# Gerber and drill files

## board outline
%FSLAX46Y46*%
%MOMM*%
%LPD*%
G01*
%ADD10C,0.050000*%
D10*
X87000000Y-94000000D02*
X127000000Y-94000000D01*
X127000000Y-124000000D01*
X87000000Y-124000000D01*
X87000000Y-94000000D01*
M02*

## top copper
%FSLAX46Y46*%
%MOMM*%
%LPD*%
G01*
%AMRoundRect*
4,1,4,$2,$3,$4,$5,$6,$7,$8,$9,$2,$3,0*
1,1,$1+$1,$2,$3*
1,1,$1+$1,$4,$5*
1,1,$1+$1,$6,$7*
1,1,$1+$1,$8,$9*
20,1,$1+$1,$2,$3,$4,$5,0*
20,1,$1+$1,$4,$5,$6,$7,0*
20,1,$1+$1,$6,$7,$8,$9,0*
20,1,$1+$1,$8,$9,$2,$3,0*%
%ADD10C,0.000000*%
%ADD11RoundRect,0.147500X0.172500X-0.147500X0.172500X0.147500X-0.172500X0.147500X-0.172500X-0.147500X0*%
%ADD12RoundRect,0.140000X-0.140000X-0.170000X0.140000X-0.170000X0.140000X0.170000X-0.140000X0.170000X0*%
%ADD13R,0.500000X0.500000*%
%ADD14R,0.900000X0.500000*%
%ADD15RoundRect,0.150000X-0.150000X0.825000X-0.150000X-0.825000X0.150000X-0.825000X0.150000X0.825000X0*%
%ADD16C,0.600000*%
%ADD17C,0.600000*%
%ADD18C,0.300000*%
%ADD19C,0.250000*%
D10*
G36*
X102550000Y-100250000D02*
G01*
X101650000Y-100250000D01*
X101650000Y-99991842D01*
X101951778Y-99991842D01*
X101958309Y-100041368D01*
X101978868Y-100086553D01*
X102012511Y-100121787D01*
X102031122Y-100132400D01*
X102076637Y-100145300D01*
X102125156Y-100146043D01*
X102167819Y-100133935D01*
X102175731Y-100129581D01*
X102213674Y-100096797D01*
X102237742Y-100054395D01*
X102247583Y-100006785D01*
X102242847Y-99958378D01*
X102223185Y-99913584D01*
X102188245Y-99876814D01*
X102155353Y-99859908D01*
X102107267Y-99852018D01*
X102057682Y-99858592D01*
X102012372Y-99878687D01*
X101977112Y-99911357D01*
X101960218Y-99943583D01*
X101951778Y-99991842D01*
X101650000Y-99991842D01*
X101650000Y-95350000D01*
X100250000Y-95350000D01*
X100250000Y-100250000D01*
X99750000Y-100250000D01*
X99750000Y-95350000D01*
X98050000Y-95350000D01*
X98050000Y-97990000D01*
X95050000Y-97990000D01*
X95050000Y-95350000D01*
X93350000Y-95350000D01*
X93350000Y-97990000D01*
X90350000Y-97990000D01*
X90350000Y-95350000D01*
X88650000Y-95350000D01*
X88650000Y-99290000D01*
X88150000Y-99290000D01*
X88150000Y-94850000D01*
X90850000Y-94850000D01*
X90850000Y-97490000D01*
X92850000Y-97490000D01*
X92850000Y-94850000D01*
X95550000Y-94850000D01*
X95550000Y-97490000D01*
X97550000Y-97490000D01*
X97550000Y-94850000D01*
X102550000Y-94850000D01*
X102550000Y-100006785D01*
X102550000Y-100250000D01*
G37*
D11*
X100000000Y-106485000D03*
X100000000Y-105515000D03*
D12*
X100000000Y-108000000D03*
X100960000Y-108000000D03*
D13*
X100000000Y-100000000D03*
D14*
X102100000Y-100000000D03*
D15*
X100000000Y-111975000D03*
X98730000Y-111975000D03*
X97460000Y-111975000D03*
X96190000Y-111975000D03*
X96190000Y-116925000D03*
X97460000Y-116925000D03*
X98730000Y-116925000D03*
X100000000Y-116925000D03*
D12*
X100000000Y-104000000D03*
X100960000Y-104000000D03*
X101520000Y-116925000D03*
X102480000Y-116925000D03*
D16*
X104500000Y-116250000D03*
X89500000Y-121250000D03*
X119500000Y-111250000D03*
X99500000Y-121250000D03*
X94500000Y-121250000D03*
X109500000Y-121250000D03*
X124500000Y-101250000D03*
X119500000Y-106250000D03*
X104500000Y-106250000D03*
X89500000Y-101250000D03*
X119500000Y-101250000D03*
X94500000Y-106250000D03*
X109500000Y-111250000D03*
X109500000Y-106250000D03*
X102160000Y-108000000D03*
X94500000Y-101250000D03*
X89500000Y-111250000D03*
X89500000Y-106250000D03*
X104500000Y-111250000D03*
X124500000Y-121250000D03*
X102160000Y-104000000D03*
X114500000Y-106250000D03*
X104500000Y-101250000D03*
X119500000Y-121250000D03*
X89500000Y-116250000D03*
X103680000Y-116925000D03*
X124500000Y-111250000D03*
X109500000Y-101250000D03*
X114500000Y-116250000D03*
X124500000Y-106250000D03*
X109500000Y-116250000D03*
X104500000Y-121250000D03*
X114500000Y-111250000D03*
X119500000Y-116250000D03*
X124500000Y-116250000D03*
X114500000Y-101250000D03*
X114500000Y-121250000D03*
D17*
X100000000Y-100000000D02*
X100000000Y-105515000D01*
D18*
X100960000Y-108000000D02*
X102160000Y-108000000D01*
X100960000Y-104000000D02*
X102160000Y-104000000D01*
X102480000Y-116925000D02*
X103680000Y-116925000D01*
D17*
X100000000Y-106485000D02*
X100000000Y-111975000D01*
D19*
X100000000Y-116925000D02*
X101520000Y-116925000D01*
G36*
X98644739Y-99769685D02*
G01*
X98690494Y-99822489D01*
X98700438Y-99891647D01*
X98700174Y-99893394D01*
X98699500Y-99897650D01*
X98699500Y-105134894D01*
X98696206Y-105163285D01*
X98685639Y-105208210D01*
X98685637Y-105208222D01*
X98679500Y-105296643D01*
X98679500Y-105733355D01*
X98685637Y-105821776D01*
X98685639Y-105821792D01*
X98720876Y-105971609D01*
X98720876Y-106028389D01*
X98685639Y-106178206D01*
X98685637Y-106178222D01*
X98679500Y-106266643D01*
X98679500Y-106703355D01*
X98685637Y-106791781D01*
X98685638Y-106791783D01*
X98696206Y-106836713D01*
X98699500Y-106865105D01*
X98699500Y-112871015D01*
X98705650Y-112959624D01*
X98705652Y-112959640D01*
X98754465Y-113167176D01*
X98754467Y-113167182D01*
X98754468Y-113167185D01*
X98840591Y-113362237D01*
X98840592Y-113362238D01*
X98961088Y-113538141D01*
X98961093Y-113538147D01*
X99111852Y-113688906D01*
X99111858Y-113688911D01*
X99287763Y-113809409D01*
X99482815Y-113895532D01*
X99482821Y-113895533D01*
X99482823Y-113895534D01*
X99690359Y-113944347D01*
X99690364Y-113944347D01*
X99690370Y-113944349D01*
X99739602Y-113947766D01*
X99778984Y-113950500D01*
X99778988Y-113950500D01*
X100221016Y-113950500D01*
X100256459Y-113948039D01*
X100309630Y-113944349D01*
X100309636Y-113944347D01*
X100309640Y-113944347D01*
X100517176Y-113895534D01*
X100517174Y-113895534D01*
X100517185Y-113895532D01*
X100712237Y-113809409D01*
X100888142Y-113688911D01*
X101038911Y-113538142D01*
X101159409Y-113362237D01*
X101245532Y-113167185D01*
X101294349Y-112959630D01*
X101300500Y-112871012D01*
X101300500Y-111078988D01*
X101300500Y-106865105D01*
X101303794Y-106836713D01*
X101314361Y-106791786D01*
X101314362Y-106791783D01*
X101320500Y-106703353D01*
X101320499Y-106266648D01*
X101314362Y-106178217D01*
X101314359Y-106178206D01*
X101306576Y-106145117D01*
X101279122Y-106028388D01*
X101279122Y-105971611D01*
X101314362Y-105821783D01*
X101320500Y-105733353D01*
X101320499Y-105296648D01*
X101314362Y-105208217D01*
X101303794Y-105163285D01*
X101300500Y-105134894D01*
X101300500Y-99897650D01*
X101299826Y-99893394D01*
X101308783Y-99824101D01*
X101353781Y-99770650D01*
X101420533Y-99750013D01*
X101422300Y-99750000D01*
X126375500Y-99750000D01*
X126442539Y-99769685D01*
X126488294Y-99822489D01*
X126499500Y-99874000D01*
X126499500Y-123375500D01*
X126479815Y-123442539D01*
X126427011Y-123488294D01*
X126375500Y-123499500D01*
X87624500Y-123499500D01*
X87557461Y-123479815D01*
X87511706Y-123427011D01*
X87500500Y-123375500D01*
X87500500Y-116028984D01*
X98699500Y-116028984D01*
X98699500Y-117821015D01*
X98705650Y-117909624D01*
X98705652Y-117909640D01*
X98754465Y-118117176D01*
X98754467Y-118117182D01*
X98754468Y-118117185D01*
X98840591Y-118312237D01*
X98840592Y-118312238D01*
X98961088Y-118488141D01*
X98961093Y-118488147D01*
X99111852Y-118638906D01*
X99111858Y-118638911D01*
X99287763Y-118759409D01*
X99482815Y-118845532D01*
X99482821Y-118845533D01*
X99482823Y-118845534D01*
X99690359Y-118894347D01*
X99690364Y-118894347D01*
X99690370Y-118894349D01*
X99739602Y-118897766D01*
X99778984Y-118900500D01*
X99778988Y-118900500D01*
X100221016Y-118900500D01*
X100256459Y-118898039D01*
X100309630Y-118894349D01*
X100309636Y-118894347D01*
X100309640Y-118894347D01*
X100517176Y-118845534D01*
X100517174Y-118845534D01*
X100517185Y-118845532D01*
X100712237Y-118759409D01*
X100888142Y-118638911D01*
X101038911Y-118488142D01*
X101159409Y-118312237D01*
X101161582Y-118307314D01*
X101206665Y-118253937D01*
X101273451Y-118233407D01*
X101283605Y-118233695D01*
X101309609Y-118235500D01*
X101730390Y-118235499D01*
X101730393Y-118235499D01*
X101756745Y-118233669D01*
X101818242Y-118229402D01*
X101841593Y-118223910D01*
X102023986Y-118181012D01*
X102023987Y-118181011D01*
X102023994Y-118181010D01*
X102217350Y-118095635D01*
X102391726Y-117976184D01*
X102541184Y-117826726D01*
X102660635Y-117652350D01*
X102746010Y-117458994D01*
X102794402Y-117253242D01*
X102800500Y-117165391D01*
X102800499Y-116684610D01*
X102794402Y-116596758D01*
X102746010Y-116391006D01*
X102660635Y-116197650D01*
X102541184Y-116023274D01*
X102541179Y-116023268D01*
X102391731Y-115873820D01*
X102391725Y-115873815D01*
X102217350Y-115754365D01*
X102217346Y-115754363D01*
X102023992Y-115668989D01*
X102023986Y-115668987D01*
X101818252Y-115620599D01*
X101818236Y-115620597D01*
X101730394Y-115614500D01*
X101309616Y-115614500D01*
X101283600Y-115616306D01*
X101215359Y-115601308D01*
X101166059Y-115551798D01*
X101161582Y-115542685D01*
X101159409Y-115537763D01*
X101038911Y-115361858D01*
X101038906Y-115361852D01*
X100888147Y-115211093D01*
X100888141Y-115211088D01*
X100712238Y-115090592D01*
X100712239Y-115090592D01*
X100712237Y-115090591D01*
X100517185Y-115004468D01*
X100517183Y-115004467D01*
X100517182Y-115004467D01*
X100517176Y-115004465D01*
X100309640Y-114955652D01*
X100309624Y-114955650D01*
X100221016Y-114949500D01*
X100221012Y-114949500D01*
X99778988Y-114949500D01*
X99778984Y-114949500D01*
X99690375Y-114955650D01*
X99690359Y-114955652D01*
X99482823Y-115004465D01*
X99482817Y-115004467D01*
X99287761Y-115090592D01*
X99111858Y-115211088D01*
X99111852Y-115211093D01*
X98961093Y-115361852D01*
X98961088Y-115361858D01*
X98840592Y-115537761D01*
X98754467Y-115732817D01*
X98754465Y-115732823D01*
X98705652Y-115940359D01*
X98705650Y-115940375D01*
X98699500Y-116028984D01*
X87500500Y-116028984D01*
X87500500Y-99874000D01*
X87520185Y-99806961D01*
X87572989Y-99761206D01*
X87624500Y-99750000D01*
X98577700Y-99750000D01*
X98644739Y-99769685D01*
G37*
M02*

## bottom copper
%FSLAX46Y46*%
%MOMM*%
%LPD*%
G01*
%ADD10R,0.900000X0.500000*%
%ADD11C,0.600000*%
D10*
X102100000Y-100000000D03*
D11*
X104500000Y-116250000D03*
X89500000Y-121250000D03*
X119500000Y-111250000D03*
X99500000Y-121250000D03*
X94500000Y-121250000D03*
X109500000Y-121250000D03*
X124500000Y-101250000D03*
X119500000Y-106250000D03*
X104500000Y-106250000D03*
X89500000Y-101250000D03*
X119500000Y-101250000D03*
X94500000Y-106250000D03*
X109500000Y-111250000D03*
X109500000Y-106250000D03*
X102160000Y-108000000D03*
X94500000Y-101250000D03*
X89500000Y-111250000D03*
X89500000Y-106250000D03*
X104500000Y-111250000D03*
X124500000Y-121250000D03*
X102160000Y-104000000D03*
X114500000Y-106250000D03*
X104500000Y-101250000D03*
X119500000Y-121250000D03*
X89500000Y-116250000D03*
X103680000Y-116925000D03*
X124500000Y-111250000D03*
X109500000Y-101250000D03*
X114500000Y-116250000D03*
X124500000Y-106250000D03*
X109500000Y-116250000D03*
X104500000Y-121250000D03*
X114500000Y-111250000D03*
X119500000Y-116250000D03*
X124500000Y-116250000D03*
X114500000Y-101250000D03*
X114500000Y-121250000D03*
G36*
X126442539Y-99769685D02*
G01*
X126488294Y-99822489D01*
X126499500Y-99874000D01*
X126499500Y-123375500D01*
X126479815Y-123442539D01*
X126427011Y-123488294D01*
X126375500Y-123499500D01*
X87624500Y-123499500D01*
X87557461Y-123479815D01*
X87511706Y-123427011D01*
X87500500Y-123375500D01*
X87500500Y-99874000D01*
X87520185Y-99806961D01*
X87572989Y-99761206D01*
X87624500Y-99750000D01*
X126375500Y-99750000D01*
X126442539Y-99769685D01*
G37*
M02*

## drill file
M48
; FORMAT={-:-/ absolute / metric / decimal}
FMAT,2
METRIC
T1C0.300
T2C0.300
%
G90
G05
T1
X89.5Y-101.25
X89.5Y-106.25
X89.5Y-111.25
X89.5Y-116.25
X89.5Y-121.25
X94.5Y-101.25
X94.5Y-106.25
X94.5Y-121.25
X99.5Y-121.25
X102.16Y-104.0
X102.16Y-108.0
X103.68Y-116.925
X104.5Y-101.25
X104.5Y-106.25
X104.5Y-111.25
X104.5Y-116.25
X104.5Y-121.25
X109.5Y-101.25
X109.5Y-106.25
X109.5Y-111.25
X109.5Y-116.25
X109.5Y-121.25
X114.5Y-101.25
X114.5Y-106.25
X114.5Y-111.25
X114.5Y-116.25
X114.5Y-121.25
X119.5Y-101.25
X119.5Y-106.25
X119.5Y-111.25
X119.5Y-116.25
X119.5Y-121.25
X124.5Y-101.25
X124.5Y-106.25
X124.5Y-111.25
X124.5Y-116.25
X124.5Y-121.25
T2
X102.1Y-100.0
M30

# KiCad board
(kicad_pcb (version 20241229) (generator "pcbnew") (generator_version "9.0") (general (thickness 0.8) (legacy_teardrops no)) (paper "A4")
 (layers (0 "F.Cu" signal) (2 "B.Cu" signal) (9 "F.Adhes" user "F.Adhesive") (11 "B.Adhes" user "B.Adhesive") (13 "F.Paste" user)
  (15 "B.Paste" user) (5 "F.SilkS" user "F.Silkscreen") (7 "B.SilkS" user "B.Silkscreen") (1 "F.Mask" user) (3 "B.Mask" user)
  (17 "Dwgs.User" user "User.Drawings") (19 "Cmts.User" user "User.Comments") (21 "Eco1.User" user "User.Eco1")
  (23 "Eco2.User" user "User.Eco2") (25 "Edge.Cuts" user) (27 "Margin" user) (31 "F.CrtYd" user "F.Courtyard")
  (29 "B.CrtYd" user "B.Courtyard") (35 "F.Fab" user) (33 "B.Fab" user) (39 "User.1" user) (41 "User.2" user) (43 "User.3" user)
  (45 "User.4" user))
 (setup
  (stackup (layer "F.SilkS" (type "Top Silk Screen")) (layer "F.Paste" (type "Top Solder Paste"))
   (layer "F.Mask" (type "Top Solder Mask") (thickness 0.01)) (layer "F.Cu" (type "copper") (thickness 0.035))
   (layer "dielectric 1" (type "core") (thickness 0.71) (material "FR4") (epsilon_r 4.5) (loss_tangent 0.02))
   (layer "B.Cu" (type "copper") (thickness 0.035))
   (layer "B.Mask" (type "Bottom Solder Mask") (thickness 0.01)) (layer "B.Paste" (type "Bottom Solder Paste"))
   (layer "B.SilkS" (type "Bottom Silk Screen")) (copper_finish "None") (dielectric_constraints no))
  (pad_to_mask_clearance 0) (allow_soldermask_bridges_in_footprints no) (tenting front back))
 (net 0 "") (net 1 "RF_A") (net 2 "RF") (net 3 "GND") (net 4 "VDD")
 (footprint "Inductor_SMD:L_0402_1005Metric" (layer "F.Cu") (at 100 106 90)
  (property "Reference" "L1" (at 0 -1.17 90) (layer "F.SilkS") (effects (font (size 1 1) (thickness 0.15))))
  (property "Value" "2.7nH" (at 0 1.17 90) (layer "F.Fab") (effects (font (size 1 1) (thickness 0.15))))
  (pad "1" smd roundrect (at -0.485 0 90) (size 0.59 0.64) (layers "F.Cu" "F.Mask" "F.Paste") (roundrect_rratio 0.25) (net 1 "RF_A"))
  (pad "2" smd roundrect (at 0.485 0 90) (size 0.59 0.64) (layers "F.Cu" "F.Mask" "F.Paste") (roundrect_rratio 0.25) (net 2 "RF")))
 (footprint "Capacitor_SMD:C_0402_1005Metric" (layer "F.Cu") (at 100.48 108)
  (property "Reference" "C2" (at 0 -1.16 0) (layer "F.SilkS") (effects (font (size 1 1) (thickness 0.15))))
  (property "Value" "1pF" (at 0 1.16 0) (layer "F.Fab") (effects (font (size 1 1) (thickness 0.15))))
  (pad "1" smd roundrect (at -0.48 0) (size 0.56 0.62) (layers "F.Cu" "F.Mask" "F.Paste") (roundrect_rratio 0.25) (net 1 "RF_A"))
  (pad "2" smd roundrect (at 0.48 0) (size 0.56 0.62) (layers "F.Cu" "F.Mask" "F.Paste") (roundrect_rratio 0.25) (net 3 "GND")))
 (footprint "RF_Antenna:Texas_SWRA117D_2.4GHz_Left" (layer "F.Cu") (at 100 100)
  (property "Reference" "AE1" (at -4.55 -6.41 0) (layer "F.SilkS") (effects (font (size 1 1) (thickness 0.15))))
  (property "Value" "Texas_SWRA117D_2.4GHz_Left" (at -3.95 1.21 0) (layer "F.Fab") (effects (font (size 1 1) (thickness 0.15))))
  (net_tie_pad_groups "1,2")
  (fp_poly
   (pts (xy -2.45 -2.51) (xy -4.45 -2.51) (xy -4.45 -5.15) (xy -7.15 -5.15) (xy -7.15 -2.51) (xy -9.15 -2.51) (xy -9.15 -5.15)
    (xy -11.85 -5.15) (xy -11.85 -0.71) (xy -11.35 -0.71) (xy -11.35 -4.65) (xy -9.65 -4.65) (xy -9.65 -2.01) (xy -6.65 -2.01)
    (xy -6.65 -4.65) (xy -4.95 -4.65) (xy -4.95 -2.01) (xy -1.95 -2.01) (xy -1.95 -4.65) (xy -0.25 -4.65) (xy -0.25 0.25) (xy 0.25 0.25)
    (xy 0.25 -4.65) (xy 1.65 -4.65) (xy 1.65 0.25) (xy 2.55 0.25) (xy 2.55 0.006785) (xy 2.247583 0.006785) (xy 2.237742 0.054395)
    (xy 2.213674 0.096797) (xy 2.175731 0.129581) (xy 2.167819 0.133935) (xy 2.125156 0.146043) (xy 2.076637 0.1453) (xy 2.031122 0.1324)
    (xy 2.012511 0.121787) (xy 1.978868 0.086553) (xy 1.958309 0.041368) (xy 1.951778 -0.008158) (xy 1.960218 -0.056417)
    (xy 1.977112 -0.088643) (xy 2.012372 -0.121313) (xy 2.057682 -0.141408) (xy 2.107267 -0.147982) (xy 2.155353 -0.140092)
    (xy 2.188245 -0.123186) (xy 2.223185 -0.086416) (xy 2.242847 -0.041622) (xy 2.247583 0.006785) (xy 2.55 0.006785) (xy 2.55 -5.15)
    (xy -2.45 -5.15) (xy -2.45 -2.51))
   (stroke (width 0) (type solid)) (fill yes) (layer "F.Cu"))
  (pad "1" connect rect (at 0 0) (size 0.5 0.5) (layers "F.Cu") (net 2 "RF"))
  (pad "2" thru_hole rect (at 2.1 0) (size 0.9 0.5) (drill 0.3) (layers "*.Cu") (remove_unused_layers no) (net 3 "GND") (zone_connect 2)))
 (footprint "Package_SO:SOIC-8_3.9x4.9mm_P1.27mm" (layer "F.Cu") (at 98.095 114.45 -90)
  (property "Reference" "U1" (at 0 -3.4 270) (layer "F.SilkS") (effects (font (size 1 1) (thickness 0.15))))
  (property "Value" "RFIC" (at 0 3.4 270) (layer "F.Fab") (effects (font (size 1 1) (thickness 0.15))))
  (pad "1" smd roundrect (at -2.475 -1.905 270) (size 1.95 0.6) (layers "F.Cu" "F.Mask" "F.Paste") (roundrect_rratio 0.25) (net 1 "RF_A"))
  (pad "2" smd roundrect (at -2.475 -0.635 270) (size 1.95 0.6) (layers "F.Cu" "F.Mask" "F.Paste") (roundrect_rratio 0.25) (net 3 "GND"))
  (pad "3" smd roundrect (at -2.475 0.635 270) (size 1.95 0.6) (layers "F.Cu" "F.Mask" "F.Paste") (roundrect_rratio 0.25) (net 3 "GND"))
  (pad "4" smd roundrect (at -2.475 1.905 270) (size 1.95 0.6) (layers "F.Cu" "F.Mask" "F.Paste") (roundrect_rratio 0.25) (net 3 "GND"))
  (pad "5" smd roundrect (at 2.475 1.905 270) (size 1.95 0.6) (layers "F.Cu" "F.Mask" "F.Paste") (roundrect_rratio 0.25) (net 3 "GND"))
  (pad "6" smd roundrect (at 2.475 0.635 270) (size 1.95 0.6) (layers "F.Cu" "F.Mask" "F.Paste") (roundrect_rratio 0.25) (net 3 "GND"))
  (pad "7" smd roundrect (at 2.475 -0.635 270) (size 1.95 0.6) (layers "F.Cu" "F.Mask" "F.Paste") (roundrect_rratio 0.25) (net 3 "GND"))
  (pad "8" smd roundrect (at 2.475 -1.905 270) (size 1.95 0.6) (layers "F.Cu" "F.Mask" "F.Paste") (roundrect_rratio 0.25) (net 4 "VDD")))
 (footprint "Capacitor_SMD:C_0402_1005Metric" (layer "F.Cu") (at 100.48 104)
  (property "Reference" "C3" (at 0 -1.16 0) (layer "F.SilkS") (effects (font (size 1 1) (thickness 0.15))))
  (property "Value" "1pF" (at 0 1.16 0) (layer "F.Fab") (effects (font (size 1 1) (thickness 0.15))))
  (pad "1" smd roundrect (at -0.48 0) (size 0.56 0.62) (layers "F.Cu" "F.Mask" "F.Paste") (roundrect_rratio 0.25) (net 2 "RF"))
  (pad "2" smd roundrect (at 0.48 0) (size 0.56 0.62) (layers "F.Cu" "F.Mask" "F.Paste") (roundrect_rratio 0.25) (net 3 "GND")))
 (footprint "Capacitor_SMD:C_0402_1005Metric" (layer "F.Cu") (at 102 116.925)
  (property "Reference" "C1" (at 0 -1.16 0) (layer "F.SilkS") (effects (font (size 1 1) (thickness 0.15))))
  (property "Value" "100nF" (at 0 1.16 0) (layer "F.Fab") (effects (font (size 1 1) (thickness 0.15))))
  (pad "1" smd roundrect (at -0.48 0) (size 0.56 0.62) (layers "F.Cu" "F.Mask" "F.Paste") (roundrect_rratio 0.25) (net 4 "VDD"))
  (pad "2" smd roundrect (at 0.48 0) (size 0.56 0.62) (layers "F.Cu" "F.Mask" "F.Paste") (roundrect_rratio 0.25) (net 3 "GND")))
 (gr_rect (start 87 94) (end 127 124) (stroke (width 0.05) (type default)) (fill no) (layer "Edge.Cuts"))
 (segment (start 100 100) (end 100 105.515) (width 0.6) (layer "F.Cu") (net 2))
 (segment (start 100.96 108) (end 102.16 108) (width 0.3) (layer "F.Cu") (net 3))
 (segment (start 100.96 104) (end 102.16 104) (width 0.3) (layer "F.Cu") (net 3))
 (segment (start 102.48 116.925) (end 103.68 116.925) (width 0.3) (layer "F.Cu") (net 3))
 (via (at 104.5 116.25) (size 0.6) (drill 0.3) (layers "F.Cu" "B.Cu") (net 3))
 (via (at 89.5 121.25) (size 0.6) (drill 0.3) (layers "F.Cu" "B.Cu") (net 3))
 (via (at 119.5 111.25) (size 0.6) (drill 0.3) (layers "F.Cu" "B.Cu") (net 3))
 (via (at 99.5 121.25) (size 0.6) (drill 0.3) (layers "F.Cu" "B.Cu") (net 3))
 (via (at 94.5 121.25) (size 0.6) (drill 0.3) (layers "F.Cu" "B.Cu") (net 3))
 (via (at 109.5 121.25) (size 0.6) (drill 0.3) (layers "F.Cu" "B.Cu") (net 3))
 (via (at 124.5 101.25) (size 0.6) (drill 0.3) (layers "F.Cu" "B.Cu") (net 3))
 (via (at 119.5 106.25) (size 0.6) (drill 0.3) (layers "F.Cu" "B.Cu") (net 3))
 (via (at 104.5 106.25) (size 0.6) (drill 0.3) (layers "F.Cu" "B.Cu") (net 3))
 (via (at 89.5 101.25) (size 0.6) (drill 0.3) (layers "F.Cu" "B.Cu") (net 3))
 (via (at 119.5 101.25) (size 0.6) (drill 0.3) (layers "F.Cu" "B.Cu") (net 3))
 (via (at 94.5 106.25) (size 0.6) (drill 0.3) (layers "F.Cu" "B.Cu") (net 3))
 (via (at 109.5 111.25) (size 0.6) (drill 0.3) (layers "F.Cu" "B.Cu") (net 3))
 (via (at 109.5 106.25) (size 0.6) (drill 0.3) (layers "F.Cu" "B.Cu") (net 3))
 (via (at 102.16 108) (size 0.6) (drill 0.3) (layers "F.Cu" "B.Cu") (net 3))
 (via (at 94.5 101.25) (size 0.6) (drill 0.3) (layers "F.Cu" "B.Cu") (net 3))
 (via (at 89.5 111.25) (size 0.6) (drill 0.3) (layers "F.Cu" "B.Cu") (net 3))
 (via (at 89.5 106.25) (size 0.6) (drill 0.3) (layers "F.Cu" "B.Cu") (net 3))
 (via (at 104.5 111.25) (size 0.6) (drill 0.3) (layers "F.Cu" "B.Cu") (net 3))
 (via (at 124.5 121.25) (size 0.6) (drill 0.3) (layers "F.Cu" "B.Cu") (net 3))
 (via (at 102.16 104) (size 0.6) (drill 0.3) (layers "F.Cu" "B.Cu") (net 3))
 (via (at 114.5 106.25) (size 0.6) (drill 0.3) (layers "F.Cu" "B.Cu") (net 3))
 (via (at 104.5 101.25) (size 0.6) (drill 0.3) (layers "F.Cu" "B.Cu") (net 3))
 (via (at 119.5 121.25) (size 0.6) (drill 0.3) (layers "F.Cu" "B.Cu") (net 3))
 (via (at 89.5 116.25) (size 0.6) (drill 0.3) (layers "F.Cu" "B.Cu") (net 3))
 (via (at 103.68 116.925) (size 0.6) (drill 0.3) (layers "F.Cu" "B.Cu") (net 3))
 (via (at 124.5 111.25) (size 0.6) (drill 0.3) (layers "F.Cu" "B.Cu") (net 3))
 (via (at 109.5 101.25) (size 0.6) (drill 0.3) (layers "F.Cu" "B.Cu") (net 3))
 (via (at 114.5 116.25) (size 0.6) (drill 0.3) (layers "F.Cu" "B.Cu") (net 3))
 (via (at 124.5 106.25) (size 0.6) (drill 0.3) (layers "F.Cu" "B.Cu") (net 3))
 (via (at 109.5 116.25) (size 0.6) (drill 0.3) (layers "F.Cu" "B.Cu") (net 3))
 (via (at 104.5 121.25) (size 0.6) (drill 0.3) (layers "F.Cu" "B.Cu") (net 3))
 (via (at 114.5 111.25) (size 0.6) (drill 0.3) (layers "F.Cu" "B.Cu") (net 3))
 (via (at 119.5 116.25) (size 0.6) (drill 0.3) (layers "F.Cu" "B.Cu") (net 3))
 (via (at 124.5 116.25) (size 0.6) (drill 0.3) (layers "F.Cu" "B.Cu") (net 3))
 (via (at 114.5 101.25) (size 0.6) (drill 0.3) (layers "F.Cu" "B.Cu") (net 3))
 (via (at 114.5 121.25) (size 0.6) (drill 0.3) (layers "F.Cu" "B.Cu") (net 3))
 (segment (start 100 106.485) (end 100 111.975) (width 0.6) (layer "F.Cu") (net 1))
 (segment (start 100 116.925) (end 101.52 116.925) (width 0.25) (layer "F.Cu") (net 4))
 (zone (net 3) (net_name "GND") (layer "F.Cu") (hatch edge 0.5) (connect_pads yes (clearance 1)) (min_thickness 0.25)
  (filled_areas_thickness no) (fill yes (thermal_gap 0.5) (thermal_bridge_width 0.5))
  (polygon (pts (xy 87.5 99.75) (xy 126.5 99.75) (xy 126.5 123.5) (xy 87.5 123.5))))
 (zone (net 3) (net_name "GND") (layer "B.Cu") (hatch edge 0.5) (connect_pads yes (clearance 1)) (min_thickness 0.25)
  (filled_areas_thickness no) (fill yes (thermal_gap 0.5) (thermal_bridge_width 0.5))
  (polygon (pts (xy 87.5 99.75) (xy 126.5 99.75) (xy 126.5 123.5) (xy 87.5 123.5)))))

